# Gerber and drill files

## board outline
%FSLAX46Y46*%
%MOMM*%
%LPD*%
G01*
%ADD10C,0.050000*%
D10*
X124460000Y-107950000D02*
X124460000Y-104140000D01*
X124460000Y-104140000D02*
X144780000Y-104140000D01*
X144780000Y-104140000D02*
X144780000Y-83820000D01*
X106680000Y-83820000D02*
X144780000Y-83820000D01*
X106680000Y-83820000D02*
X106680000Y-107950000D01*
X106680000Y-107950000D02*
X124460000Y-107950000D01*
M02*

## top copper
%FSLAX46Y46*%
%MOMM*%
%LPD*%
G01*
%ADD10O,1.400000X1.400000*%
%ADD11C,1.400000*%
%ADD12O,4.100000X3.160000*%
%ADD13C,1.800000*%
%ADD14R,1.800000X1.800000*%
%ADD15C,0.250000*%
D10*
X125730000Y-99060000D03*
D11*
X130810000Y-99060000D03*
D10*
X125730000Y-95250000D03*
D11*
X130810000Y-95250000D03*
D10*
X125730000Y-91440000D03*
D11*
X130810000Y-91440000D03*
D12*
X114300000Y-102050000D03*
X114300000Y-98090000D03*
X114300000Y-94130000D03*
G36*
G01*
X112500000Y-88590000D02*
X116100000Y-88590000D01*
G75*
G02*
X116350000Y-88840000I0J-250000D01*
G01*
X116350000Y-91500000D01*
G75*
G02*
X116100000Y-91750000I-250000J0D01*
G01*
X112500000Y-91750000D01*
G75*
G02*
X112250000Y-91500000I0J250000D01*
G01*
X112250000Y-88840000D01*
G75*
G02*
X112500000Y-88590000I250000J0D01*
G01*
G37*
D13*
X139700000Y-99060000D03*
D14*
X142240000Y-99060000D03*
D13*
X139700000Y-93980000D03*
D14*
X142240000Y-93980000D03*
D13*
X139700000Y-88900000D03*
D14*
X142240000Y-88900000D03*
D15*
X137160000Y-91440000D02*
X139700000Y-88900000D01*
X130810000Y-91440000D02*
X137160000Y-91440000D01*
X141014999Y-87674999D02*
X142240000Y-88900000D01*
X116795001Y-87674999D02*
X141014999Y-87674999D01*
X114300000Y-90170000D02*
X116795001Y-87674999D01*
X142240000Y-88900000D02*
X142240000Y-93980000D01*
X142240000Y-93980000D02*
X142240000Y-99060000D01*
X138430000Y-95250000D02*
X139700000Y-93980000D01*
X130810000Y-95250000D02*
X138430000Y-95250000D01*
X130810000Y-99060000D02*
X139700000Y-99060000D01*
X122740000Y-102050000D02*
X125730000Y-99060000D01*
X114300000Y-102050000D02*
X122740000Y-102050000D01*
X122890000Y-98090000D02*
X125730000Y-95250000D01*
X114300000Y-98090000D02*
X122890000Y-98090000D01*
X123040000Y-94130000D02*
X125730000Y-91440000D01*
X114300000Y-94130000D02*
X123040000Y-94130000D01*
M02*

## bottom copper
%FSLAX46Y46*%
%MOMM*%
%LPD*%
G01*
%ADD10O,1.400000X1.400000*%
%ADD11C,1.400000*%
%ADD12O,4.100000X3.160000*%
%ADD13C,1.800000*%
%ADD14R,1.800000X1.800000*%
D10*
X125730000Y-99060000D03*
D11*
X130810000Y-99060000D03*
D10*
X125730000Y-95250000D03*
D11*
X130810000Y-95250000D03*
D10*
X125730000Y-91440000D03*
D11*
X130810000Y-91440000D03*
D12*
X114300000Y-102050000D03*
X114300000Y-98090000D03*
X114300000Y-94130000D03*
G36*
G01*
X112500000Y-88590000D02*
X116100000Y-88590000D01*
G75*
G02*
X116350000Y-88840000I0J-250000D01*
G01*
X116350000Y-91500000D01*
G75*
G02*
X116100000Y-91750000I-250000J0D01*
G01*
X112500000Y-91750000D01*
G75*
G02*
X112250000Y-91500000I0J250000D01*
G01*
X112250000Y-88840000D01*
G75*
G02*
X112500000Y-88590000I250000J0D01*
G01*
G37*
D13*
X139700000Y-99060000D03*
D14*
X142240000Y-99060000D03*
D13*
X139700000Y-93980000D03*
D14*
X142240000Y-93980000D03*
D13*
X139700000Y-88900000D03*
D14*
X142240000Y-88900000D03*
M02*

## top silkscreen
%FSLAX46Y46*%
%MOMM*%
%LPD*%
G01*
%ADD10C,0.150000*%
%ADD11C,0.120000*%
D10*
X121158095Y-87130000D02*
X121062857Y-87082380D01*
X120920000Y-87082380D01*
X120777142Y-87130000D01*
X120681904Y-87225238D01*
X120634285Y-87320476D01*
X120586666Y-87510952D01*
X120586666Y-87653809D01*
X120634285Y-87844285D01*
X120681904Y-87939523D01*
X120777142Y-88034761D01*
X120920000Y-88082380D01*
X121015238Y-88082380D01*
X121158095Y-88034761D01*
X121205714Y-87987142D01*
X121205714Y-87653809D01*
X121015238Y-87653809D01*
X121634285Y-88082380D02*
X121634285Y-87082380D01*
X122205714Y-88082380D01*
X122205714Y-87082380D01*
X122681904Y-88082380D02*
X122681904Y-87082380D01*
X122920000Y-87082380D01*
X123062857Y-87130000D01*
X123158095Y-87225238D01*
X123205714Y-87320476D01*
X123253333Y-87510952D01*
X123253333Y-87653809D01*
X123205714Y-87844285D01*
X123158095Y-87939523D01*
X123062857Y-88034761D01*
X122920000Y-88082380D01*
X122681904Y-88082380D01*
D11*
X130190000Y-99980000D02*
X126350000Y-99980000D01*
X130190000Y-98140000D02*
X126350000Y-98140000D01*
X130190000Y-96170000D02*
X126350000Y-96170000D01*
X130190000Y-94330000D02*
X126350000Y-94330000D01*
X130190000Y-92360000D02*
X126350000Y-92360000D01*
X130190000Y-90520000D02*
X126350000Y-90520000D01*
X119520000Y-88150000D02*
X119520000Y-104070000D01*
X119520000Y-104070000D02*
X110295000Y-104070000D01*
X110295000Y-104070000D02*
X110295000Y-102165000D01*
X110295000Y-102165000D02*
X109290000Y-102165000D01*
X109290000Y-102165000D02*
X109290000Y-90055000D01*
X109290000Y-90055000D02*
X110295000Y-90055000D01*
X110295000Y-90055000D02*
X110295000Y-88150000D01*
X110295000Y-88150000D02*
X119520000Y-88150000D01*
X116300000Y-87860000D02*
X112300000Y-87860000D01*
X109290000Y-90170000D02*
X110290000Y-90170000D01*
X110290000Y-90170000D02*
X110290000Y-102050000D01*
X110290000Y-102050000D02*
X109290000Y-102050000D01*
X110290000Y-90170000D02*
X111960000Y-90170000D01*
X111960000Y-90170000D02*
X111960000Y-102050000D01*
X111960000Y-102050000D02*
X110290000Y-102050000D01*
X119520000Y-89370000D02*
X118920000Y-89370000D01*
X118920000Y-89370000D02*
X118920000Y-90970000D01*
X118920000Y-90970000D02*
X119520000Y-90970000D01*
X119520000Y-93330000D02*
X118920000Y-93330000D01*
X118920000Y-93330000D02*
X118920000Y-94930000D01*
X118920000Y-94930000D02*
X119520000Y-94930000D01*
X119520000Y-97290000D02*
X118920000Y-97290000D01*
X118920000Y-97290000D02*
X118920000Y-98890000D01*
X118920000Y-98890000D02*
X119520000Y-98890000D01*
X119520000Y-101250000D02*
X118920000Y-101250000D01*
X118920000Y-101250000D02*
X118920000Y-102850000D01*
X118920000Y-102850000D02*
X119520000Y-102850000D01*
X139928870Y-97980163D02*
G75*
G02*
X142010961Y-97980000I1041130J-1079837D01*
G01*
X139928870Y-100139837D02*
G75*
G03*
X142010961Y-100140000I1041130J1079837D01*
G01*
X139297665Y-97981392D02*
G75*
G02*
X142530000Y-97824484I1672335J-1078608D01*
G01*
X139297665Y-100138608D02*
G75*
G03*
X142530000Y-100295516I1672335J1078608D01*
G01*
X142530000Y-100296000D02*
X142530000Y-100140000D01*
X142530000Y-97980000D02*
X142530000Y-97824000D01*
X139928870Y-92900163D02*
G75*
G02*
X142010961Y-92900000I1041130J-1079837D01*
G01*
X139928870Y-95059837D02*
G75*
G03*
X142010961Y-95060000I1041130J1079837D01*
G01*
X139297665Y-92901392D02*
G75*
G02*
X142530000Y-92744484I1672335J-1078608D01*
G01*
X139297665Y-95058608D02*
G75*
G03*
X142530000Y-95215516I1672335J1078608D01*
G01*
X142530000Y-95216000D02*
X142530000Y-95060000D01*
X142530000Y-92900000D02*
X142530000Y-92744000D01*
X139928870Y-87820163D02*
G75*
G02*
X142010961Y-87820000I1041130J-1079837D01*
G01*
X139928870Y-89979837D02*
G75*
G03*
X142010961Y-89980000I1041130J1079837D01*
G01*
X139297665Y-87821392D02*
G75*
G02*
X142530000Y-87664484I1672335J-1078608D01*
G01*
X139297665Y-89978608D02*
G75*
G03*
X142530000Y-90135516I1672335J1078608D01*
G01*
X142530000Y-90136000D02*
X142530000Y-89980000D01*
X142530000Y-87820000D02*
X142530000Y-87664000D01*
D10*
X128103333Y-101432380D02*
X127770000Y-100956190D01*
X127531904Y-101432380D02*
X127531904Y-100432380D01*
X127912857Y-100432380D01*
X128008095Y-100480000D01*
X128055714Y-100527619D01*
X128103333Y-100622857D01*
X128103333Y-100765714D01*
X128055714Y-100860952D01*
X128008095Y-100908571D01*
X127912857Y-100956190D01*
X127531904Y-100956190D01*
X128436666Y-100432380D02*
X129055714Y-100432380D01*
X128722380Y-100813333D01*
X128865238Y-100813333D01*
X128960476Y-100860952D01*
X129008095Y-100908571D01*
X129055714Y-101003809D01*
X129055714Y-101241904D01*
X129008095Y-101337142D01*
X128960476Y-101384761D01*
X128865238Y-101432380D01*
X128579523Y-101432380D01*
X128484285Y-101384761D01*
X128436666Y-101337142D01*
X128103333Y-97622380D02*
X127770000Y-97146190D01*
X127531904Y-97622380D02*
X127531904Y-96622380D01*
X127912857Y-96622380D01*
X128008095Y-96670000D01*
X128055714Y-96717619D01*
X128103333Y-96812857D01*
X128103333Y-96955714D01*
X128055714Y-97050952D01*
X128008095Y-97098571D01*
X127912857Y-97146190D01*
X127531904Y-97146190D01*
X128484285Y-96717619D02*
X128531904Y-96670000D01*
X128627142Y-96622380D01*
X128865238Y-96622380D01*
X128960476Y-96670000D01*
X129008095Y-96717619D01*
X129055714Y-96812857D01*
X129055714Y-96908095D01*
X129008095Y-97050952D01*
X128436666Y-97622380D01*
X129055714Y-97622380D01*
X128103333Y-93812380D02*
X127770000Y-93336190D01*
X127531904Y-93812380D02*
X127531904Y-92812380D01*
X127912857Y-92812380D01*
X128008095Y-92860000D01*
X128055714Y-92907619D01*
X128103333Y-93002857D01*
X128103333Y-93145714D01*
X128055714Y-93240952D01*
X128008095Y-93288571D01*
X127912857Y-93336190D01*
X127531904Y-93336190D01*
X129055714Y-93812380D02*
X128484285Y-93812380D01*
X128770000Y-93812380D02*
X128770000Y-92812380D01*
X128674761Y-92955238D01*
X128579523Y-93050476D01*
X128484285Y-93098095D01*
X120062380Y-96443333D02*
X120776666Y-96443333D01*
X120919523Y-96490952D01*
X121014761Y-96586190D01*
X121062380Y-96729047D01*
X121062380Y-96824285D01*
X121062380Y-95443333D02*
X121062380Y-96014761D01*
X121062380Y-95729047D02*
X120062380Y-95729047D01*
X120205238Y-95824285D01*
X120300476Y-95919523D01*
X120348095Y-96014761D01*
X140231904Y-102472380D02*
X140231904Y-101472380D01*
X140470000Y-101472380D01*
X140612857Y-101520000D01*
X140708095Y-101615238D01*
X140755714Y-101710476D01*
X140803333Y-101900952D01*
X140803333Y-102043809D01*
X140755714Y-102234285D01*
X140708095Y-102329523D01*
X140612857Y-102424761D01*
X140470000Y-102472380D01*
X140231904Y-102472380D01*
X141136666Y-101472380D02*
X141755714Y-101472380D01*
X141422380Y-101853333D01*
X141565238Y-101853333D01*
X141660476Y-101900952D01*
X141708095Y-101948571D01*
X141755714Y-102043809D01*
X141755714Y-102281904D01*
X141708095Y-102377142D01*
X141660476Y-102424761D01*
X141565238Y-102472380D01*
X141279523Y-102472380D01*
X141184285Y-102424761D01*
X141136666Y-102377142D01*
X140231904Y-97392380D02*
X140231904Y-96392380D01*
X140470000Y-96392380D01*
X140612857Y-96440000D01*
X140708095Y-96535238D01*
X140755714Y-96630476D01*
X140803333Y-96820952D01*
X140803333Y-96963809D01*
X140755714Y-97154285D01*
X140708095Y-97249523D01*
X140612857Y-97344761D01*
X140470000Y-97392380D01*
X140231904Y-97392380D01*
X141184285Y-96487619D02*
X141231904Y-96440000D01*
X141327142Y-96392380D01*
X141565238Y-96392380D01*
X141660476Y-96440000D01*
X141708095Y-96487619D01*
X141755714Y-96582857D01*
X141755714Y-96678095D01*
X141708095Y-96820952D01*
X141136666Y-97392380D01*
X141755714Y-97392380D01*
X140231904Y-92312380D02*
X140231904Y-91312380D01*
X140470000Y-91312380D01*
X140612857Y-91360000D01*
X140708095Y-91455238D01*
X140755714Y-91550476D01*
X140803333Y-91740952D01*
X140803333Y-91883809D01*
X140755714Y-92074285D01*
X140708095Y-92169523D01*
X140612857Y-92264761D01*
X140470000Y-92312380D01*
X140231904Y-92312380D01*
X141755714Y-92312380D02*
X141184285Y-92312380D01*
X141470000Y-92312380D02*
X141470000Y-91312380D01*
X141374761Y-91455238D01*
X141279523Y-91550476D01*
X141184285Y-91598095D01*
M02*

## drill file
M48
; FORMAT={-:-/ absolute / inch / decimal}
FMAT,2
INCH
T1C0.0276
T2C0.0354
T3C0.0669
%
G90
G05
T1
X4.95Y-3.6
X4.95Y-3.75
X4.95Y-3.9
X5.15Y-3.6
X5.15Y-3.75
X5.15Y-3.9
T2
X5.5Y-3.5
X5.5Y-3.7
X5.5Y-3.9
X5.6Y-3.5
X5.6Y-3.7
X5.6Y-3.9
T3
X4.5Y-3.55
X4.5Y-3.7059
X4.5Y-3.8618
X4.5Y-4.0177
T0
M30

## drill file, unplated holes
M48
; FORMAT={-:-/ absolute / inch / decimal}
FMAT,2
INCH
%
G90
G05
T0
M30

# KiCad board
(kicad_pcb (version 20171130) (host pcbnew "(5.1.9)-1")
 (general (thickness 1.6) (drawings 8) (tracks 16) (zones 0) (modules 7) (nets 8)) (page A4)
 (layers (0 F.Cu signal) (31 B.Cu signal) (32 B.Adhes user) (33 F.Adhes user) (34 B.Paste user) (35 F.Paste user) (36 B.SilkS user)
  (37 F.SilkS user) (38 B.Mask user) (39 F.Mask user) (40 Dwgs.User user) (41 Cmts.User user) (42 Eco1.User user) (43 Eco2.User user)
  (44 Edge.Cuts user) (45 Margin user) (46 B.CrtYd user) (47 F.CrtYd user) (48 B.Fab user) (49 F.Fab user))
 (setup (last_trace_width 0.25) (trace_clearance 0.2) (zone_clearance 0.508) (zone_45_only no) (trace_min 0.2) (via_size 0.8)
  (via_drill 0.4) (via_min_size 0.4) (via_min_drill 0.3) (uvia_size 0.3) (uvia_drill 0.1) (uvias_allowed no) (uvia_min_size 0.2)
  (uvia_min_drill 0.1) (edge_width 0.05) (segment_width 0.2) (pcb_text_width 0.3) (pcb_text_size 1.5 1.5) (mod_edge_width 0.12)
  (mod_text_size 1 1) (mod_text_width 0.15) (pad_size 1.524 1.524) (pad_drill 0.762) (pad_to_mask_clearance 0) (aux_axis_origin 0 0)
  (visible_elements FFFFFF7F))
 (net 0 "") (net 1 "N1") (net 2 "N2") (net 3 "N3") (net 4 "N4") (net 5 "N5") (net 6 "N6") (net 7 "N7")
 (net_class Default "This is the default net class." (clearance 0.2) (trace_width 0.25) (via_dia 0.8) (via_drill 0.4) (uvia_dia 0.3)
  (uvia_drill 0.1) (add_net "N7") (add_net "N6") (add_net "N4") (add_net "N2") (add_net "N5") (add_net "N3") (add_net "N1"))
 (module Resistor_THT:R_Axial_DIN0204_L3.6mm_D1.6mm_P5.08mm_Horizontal (layer F.Cu) (at 130.81 99.06 180)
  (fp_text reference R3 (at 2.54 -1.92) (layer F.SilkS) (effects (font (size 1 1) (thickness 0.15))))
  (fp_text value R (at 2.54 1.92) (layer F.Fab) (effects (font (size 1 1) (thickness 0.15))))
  (fp_line (start 0.62 -0.92) (end 4.46 -0.92) (layer F.SilkS) (width 0.12))
  (fp_line (start 0.62 0.92) (end 4.46 0.92) (layer F.SilkS) (width 0.12))
  (pad 2 thru_hole oval (at 5.08 0 180) (size 1.4 1.4) (drill 0.7) (layers *.Cu *.Mask) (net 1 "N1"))
  (pad 1 thru_hole circle (at 0 0 180) (size 1.4 1.4) (drill 0.7) (layers *.Cu *.Mask) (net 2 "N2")))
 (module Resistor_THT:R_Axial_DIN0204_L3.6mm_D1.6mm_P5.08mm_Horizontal (layer F.Cu) (at 130.81 95.25 180)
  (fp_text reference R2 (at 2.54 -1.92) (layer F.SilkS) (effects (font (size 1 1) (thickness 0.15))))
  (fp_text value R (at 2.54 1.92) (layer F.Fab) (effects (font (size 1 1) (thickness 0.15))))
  (fp_line (start 0.62 -0.92) (end 4.46 -0.92) (layer F.SilkS) (width 0.12))
  (fp_line (start 0.62 0.92) (end 4.46 0.92) (layer F.SilkS) (width 0.12))
  (pad 2 thru_hole oval (at 5.08 0 180) (size 1.4 1.4) (drill 0.7) (layers *.Cu *.Mask) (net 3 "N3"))
  (pad 1 thru_hole circle (at 0 0 180) (size 1.4 1.4) (drill 0.7) (layers *.Cu *.Mask) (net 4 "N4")))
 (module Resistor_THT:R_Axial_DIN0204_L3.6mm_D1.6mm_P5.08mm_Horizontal (layer F.Cu) (at 130.81 91.44 180)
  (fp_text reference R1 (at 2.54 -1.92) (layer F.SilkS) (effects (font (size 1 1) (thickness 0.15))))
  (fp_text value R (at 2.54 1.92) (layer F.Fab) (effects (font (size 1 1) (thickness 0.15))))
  (fp_line (start 0.62 -0.92) (end 4.46 -0.92) (layer F.SilkS) (width 0.12))
  (fp_line (start 0.62 0.92) (end 4.46 0.92) (layer F.SilkS) (width 0.12))
  (pad 2 thru_hole oval (at 5.08 0 180) (size 1.4 1.4) (drill 0.7) (layers *.Cu *.Mask) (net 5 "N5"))
  (pad 1 thru_hole circle (at 0 0 180) (size 1.4 1.4) (drill 0.7) (layers *.Cu *.Mask) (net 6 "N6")))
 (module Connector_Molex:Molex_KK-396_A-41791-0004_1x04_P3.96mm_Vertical (layer F.Cu) (at 114.3 90.17 270)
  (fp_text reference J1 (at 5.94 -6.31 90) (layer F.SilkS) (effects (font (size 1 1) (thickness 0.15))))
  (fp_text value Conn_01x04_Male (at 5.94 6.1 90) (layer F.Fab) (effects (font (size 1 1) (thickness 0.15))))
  (fp_line (start -2.02 -5.22) (end 13.9 -5.22) (layer F.SilkS) (width 0.12))
  (fp_line (start 13.9 -5.22) (end 13.9 4.005) (layer F.SilkS) (width 0.12))
  (fp_line (start 13.9 4.005) (end 11.995 4.005) (layer F.SilkS) (width 0.12))
  (fp_line (start 11.995 4.005) (end 11.995 5.01) (layer F.SilkS) (width 0.12))
  (fp_line (start 11.995 5.01) (end -0.115 5.01) (layer F.SilkS) (width 0.12))
  (fp_line (start -0.115 5.01) (end -0.115 4.005) (layer F.SilkS) (width 0.12))
  (fp_line (start -0.115 4.005) (end -2.02 4.005) (layer F.SilkS) (width 0.12))
  (fp_line (start -2.02 4.005) (end -2.02 -5.22) (layer F.SilkS) (width 0.12))
  (fp_line (start -2.31 -2) (end -2.31 2) (layer F.SilkS) (width 0.12))
  (fp_line (start 0 5.01) (end 0 4.01) (layer F.SilkS) (width 0.12))
  (fp_line (start 0 4.01) (end 11.88 4.01) (layer F.SilkS) (width 0.12))
  (fp_line (start 11.88 4.01) (end 11.88 5.01) (layer F.SilkS) (width 0.12))
  (fp_line (start 0 4.01) (end 0 2.34) (layer F.SilkS) (width 0.12))
  (fp_line (start 0 2.34) (end 11.88 2.34) (layer F.SilkS) (width 0.12))
  (fp_line (start 11.88 2.34) (end 11.88 4.01) (layer F.SilkS) (width 0.12))
  (fp_line (start -0.8 -5.22) (end -0.8 -4.62) (layer F.SilkS) (width 0.12))
  (fp_line (start -0.8 -4.62) (end 0.8 -4.62) (layer F.SilkS) (width 0.12))
  (fp_line (start 0.8 -4.62) (end 0.8 -5.22) (layer F.SilkS) (width 0.12))
  (fp_line (start 3.16 -5.22) (end 3.16 -4.62) (layer F.SilkS) (width 0.12))
  (fp_line (start 3.16 -4.62) (end 4.76 -4.62) (layer F.SilkS) (width 0.12))
  (fp_line (start 4.76 -4.62) (end 4.76 -5.22) (layer F.SilkS) (width 0.12))
  (fp_line (start 7.12 -5.22) (end 7.12 -4.62) (layer F.SilkS) (width 0.12))
  (fp_line (start 7.12 -4.62) (end 8.72 -4.62) (layer F.SilkS) (width 0.12))
  (fp_line (start 8.72 -4.62) (end 8.72 -5.22) (layer F.SilkS) (width 0.12))
  (fp_line (start 11.08 -5.22) (end 11.08 -4.62) (layer F.SilkS) (width 0.12))
  (fp_line (start 11.08 -4.62) (end 12.68 -4.62) (layer F.SilkS) (width 0.12))
  (fp_line (start 12.68 -4.62) (end 12.68 -5.22) (layer F.SilkS) (width 0.12))
  (pad 4 thru_hole oval (at 11.88 0 270) (size 3.16 4.1) (drill 1.7) (layers *.Cu *.Mask) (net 1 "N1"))
  (pad 3 thru_hole oval (at 7.92 0 270) (size 3.16 4.1) (drill 1.7) (layers *.Cu *.Mask) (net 3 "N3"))
  (pad 2 thru_hole oval (at 3.96 0 270) (size 3.16 4.1) (drill 1.7) (layers *.Cu *.Mask) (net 5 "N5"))
  (pad 1 thru_hole roundrect (at 0 0 270) (size 3.16 4.1) (drill 1.7) (layers *.Cu *.Mask) (roundrect_rratio 0.07911392405063292)
   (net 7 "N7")))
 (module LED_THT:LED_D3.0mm (layer F.Cu) (at 142.24 99.06 180)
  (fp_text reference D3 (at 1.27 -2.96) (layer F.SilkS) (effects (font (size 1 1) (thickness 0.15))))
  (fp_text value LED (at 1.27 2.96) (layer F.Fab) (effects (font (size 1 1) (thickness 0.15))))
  (fp_arc (start 1.27 0) (end 0.229039 1.08) (angle -87.9) (layer F.SilkS) (width 0.12))
  (fp_arc (start 1.27 0) (end 0.229039 -1.08) (angle 87.9) (layer F.SilkS) (width 0.12))
  (fp_arc (start 1.27 0) (end -0.29 1.235516) (angle -108.8) (layer F.SilkS) (width 0.12))
  (fp_arc (start 1.27 0) (end -0.29 -1.235516) (angle 108.8) (layer F.SilkS) (width 0.12))
  (fp_line (start -0.29 -1.236) (end -0.29 -1.08) (layer F.SilkS) (width 0.12))
  (fp_line (start -0.29 1.08) (end -0.29 1.236) (layer F.SilkS) (width 0.12))
  (pad 2 thru_hole circle (at 2.54 0 180) (size 1.8 1.8) (drill 0.9) (layers *.Cu *.Mask) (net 2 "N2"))
  (pad 1 thru_hole rect (at 0 0 180) (size 1.8 1.8) (drill 0.9) (layers *.Cu *.Mask) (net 7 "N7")))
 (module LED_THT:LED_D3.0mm (layer F.Cu) (at 142.24 93.98 180)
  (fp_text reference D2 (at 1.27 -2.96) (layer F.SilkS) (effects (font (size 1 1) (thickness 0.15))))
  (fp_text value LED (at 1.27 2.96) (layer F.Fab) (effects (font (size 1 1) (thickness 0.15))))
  (fp_arc (start 1.27 0) (end 0.229039 1.08) (angle -87.9) (layer F.SilkS) (width 0.12))
  (fp_arc (start 1.27 0) (end 0.229039 -1.08) (angle 87.9) (layer F.SilkS) (width 0.12))
  (fp_arc (start 1.27 0) (end -0.29 1.235516) (angle -108.8) (layer F.SilkS) (width 0.12))
  (fp_arc (start 1.27 0) (end -0.29 -1.235516) (angle 108.8) (layer F.SilkS) (width 0.12))
  (fp_line (start -0.29 -1.236) (end -0.29 -1.08) (layer F.SilkS) (width 0.12))
  (fp_line (start -0.29 1.08) (end -0.29 1.236) (layer F.SilkS) (width 0.12))
  (pad 2 thru_hole circle (at 2.54 0 180) (size 1.8 1.8) (drill 0.9) (layers *.Cu *.Mask) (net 4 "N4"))
  (pad 1 thru_hole rect (at 0 0 180) (size 1.8 1.8) (drill 0.9) (layers *.Cu *.Mask) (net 7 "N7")))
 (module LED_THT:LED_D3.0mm (layer F.Cu) (at 142.24 88.9 180)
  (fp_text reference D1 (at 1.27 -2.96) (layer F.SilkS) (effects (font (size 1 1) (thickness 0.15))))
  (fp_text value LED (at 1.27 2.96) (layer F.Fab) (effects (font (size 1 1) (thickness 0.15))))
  (fp_arc (start 1.27 0) (end 0.229039 1.08) (angle -87.9) (layer F.SilkS) (width 0.12))
  (fp_arc (start 1.27 0) (end 0.229039 -1.08) (angle 87.9) (layer F.SilkS) (width 0.12))
  (fp_arc (start 1.27 0) (end -0.29 1.235516) (angle -108.8) (layer F.SilkS) (width 0.12))
  (fp_arc (start 1.27 0) (end -0.29 -1.235516) (angle 108.8) (layer F.SilkS) (width 0.12))
  (fp_line (start -0.29 -1.236) (end -0.29 -1.08) (layer F.SilkS) (width 0.12))
  (fp_line (start -0.29 1.08) (end -0.29 1.236) (layer F.SilkS) (width 0.12))
  (pad 2 thru_hole circle (at 2.54 0 180) (size 1.8 1.8) (drill 0.9) (layers *.Cu *.Mask) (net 6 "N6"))
  (pad 1 thru_hole rect (at 0 0 180) (size 1.8 1.8) (drill 0.9) (layers *.Cu *.Mask) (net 7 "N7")))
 (gr_line (start 124.46 107.95) (end 124.46 104.14) (layer Edge.Cuts) (width 0.05))
 (gr_line (start 124.46 104.14) (end 144.78 104.14) (layer Edge.Cuts) (width 0.05))
 (gr_line (start 144.78 104.14) (end 144.78 83.82) (layer Edge.Cuts) (width 0.05))
 (gr_line (start 106.68 83.82) (end 144.78 83.82) (layer Edge.Cuts) (width 0.05))
 (gr_line (start 106.68 83.82) (end 106.68 107.95) (layer Edge.Cuts) (width 0.05))
 (gr_line (start 106.68 107.95) (end 124.46 107.95) (layer Edge.Cuts) (width 0.05))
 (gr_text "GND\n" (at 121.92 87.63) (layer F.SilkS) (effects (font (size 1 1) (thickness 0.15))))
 (segment (start 137.16 91.44) (end 139.7 88.9) (width 0.25) (layer F.Cu) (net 6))
 (segment (start 130.81 91.44) (end 137.16 91.44) (width 0.25) (layer F.Cu) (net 6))
 (segment (start 141.014999 87.674999) (end 142.24 88.9) (width 0.25) (layer F.Cu) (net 7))
 (segment (start 116.795001 87.674999) (end 141.014999 87.674999) (width 0.25) (layer F.Cu) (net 7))
 (segment (start 114.3 90.17) (end 116.795001 87.674999) (width 0.25) (layer F.Cu) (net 7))
 (segment (start 142.24 88.9) (end 142.24 93.98) (width 0.25) (layer F.Cu) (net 7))
 (segment (start 142.24 93.98) (end 142.24 99.06) (width 0.25) (layer F.Cu) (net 7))
 (segment (start 138.43 95.25) (end 139.7 93.98) (width 0.25) (layer F.Cu) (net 4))
 (segment (start 130.81 95.25) (end 138.43 95.25) (width 0.25) (layer F.Cu) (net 4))
 (segment (start 130.81 99.06) (end 139.7 99.06) (width 0.25) (layer F.Cu) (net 2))
 (segment (start 122.74 102.05) (end 125.73 99.06) (width 0.25) (layer F.Cu) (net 1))
 (segment (start 114.3 102.05) (end 122.74 102.05) (width 0.25) (layer F.Cu) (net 1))
 (segment (start 122.89 98.09) (end 125.73 95.25) (width 0.25) (layer F.Cu) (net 3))
 (segment (start 114.3 98.09) (end 122.89 98.09) (width 0.25) (layer F.Cu) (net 3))
 (segment (start 123.04 94.13) (end 125.73 91.44) (width 0.25) (layer F.Cu) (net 5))
 (segment (start 114.3 94.13) (end 123.04 94.13) (width 0.25) (layer F.Cu) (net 5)))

